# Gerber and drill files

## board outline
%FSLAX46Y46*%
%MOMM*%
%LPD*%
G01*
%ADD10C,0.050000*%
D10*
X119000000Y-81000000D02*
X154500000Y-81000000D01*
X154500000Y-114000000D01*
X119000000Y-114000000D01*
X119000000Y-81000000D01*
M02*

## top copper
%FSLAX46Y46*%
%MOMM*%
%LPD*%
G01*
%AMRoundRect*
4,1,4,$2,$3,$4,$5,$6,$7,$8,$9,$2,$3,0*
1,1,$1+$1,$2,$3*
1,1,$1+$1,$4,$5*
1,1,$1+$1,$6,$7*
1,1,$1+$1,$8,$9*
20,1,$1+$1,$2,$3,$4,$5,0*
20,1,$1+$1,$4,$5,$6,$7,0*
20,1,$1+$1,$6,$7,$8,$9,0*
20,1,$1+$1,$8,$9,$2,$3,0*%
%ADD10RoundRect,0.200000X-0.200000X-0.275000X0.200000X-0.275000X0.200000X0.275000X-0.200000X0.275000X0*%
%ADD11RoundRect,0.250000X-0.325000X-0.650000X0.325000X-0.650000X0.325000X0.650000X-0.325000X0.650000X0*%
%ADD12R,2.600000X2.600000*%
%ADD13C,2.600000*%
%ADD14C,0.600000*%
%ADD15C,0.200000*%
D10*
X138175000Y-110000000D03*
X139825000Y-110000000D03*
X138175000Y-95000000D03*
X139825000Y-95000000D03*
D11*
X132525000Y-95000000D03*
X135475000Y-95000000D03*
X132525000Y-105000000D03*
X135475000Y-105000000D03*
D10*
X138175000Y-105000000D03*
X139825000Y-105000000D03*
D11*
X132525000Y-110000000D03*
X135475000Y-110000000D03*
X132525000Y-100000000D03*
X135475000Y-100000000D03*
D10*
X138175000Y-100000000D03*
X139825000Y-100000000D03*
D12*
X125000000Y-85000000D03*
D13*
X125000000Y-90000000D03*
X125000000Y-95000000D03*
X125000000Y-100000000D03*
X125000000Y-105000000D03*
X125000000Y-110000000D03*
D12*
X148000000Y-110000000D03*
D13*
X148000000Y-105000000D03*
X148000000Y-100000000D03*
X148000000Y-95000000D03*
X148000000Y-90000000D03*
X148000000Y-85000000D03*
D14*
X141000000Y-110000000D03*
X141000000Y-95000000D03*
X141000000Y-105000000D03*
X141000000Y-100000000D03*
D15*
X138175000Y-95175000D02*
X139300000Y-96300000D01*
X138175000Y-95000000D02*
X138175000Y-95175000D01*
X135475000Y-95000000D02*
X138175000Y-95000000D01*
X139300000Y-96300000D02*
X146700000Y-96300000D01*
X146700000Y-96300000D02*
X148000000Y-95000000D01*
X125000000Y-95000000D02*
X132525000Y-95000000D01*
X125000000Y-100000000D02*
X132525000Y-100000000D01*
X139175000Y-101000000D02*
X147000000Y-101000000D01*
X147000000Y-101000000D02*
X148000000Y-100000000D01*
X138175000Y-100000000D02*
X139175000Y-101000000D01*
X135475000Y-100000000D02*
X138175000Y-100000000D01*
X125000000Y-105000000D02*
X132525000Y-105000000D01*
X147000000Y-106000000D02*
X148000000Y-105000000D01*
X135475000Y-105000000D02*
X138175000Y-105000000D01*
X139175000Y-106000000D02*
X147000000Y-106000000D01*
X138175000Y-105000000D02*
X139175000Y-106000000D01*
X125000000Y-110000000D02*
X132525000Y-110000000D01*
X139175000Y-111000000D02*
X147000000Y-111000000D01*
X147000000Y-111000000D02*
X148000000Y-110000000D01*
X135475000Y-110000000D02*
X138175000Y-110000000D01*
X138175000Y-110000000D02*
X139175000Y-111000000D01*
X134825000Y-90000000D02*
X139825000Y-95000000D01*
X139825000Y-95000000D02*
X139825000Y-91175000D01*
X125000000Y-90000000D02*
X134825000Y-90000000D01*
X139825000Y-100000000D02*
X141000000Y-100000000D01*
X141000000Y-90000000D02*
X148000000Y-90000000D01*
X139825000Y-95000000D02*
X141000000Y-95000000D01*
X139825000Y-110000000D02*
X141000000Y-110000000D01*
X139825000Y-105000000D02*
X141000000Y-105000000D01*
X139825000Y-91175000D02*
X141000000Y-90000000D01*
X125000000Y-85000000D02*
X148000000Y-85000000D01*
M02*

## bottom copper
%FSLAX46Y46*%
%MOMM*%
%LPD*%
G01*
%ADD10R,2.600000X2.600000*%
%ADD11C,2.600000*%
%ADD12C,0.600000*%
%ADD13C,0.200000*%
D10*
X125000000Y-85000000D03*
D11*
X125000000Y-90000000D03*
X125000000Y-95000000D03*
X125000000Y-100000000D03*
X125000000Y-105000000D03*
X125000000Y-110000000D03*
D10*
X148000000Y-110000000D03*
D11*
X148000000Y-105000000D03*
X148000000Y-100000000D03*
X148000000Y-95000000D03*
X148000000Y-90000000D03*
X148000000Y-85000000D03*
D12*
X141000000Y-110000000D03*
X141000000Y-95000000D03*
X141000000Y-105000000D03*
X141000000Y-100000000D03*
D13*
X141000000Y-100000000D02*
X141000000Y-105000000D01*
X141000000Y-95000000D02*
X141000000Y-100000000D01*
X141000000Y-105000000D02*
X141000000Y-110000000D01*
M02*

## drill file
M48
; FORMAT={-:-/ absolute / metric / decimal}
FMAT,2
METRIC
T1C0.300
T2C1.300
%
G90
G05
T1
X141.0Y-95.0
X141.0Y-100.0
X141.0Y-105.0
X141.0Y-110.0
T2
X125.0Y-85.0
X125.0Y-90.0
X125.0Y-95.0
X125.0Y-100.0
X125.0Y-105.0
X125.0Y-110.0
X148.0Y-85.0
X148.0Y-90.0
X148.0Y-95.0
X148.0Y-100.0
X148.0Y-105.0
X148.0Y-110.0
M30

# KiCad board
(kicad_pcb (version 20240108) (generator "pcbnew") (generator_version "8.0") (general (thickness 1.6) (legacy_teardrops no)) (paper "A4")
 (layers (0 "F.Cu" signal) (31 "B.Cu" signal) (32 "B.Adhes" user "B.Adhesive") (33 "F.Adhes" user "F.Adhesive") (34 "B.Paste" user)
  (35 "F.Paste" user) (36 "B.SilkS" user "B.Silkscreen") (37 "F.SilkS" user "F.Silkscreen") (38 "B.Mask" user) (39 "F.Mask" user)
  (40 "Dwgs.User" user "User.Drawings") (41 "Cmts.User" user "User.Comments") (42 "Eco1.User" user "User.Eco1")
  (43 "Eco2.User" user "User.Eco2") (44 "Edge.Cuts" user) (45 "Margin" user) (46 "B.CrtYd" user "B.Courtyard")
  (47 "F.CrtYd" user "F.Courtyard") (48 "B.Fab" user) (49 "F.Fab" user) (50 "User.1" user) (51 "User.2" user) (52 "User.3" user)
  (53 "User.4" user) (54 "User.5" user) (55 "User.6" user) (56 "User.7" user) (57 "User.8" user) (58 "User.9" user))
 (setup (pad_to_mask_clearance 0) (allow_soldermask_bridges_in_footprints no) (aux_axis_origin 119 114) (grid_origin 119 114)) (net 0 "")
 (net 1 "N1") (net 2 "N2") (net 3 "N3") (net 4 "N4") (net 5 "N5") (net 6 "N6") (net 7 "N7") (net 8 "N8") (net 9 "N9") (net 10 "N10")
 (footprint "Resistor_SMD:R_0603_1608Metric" (layer "F.Cu") (at 139 110)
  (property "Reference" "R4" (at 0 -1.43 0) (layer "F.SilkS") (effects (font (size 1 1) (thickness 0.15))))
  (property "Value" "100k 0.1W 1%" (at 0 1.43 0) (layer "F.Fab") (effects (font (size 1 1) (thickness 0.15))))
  (pad "1" smd roundrect (at -0.825 0) (size 0.8 0.95) (layers "F.Cu" "F.Paste" "F.Mask") (roundrect_rratio 0.25) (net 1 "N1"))
  (pad "2" smd roundrect (at 0.825 0) (size 0.8 0.95) (layers "F.Cu" "F.Paste" "F.Mask") (roundrect_rratio 0.25) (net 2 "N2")))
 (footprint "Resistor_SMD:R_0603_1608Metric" (layer "F.Cu") (at 139 95)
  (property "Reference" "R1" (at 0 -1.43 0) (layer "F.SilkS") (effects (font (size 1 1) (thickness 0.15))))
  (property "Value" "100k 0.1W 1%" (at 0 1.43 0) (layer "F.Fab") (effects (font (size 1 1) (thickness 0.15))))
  (pad "1" smd roundrect (at -0.825 0) (size 0.8 0.95) (layers "F.Cu" "F.Paste" "F.Mask") (roundrect_rratio 0.25) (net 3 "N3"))
  (pad "2" smd roundrect (at 0.825 0) (size 0.8 0.95) (layers "F.Cu" "F.Paste" "F.Mask") (roundrect_rratio 0.25) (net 2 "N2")))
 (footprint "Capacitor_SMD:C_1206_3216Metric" (layer "F.Cu") (at 134 95)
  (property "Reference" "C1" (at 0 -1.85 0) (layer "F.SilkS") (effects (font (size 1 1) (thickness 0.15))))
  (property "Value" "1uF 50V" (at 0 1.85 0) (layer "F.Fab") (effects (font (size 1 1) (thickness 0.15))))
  (pad "1" smd roundrect (at -1.475 0) (size 1.15 1.8) (layers "F.Cu" "F.Paste" "F.Mask") (roundrect_rratio 0.217391) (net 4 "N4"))
  (pad "2" smd roundrect (at 1.475 0) (size 1.15 1.8) (layers "F.Cu" "F.Paste" "F.Mask") (roundrect_rratio 0.217391) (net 3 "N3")))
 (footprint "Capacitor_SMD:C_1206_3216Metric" (layer "F.Cu") (at 134 105)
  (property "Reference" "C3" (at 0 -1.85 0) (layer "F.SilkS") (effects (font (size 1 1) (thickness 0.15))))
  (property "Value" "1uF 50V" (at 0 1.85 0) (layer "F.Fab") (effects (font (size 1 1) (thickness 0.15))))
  (pad "1" smd roundrect (at -1.475 0) (size 1.15 1.8) (layers "F.Cu" "F.Paste" "F.Mask") (roundrect_rratio 0.217391) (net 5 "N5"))
  (pad "2" smd roundrect (at 1.475 0) (size 1.15 1.8) (layers "F.Cu" "F.Paste" "F.Mask") (roundrect_rratio 0.217391) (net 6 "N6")))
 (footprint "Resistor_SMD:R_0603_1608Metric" (layer "F.Cu") (at 139 105)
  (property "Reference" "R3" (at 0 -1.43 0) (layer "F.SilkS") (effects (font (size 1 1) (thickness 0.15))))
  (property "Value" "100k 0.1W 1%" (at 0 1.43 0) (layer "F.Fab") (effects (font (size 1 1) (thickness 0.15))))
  (pad "1" smd roundrect (at -0.825 0) (size 0.8 0.95) (layers "F.Cu" "F.Paste" "F.Mask") (roundrect_rratio 0.25) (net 6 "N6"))
  (pad "2" smd roundrect (at 0.825 0) (size 0.8 0.95) (layers "F.Cu" "F.Paste" "F.Mask") (roundrect_rratio 0.25) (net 2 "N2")))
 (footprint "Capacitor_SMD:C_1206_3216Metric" (layer "F.Cu") (at 134 110)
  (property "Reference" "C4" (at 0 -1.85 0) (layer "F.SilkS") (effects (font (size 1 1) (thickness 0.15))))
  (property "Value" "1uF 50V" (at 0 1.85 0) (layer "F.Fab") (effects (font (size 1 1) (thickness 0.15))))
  (pad "1" smd roundrect (at -1.475 0) (size 1.15 1.8) (layers "F.Cu" "F.Paste" "F.Mask") (roundrect_rratio 0.217391) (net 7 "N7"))
  (pad "2" smd roundrect (at 1.475 0) (size 1.15 1.8) (layers "F.Cu" "F.Paste" "F.Mask") (roundrect_rratio 0.217391) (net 1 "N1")))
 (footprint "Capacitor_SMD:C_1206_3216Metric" (layer "F.Cu") (at 134 100)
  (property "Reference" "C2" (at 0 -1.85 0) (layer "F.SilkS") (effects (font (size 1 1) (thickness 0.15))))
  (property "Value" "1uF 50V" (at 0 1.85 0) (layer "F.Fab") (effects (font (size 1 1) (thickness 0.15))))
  (pad "1" smd roundrect (at -1.475 0) (size 1.15 1.8) (layers "F.Cu" "F.Paste" "F.Mask") (roundrect_rratio 0.217391) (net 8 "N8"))
  (pad "2" smd roundrect (at 1.475 0) (size 1.15 1.8) (layers "F.Cu" "F.Paste" "F.Mask") (roundrect_rratio 0.217391) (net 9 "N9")))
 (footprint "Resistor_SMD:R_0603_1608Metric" (layer "F.Cu") (at 139 100)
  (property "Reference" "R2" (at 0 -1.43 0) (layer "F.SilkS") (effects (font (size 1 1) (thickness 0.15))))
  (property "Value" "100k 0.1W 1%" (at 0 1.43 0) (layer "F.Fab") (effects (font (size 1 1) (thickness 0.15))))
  (pad "1" smd roundrect (at -0.825 0) (size 0.8 0.95) (layers "F.Cu" "F.Paste" "F.Mask") (roundrect_rratio 0.25) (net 9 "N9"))
  (pad "2" smd roundrect (at 0.825 0) (size 0.8 0.95) (layers "F.Cu" "F.Paste" "F.Mask") (roundrect_rratio 0.25) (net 2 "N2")))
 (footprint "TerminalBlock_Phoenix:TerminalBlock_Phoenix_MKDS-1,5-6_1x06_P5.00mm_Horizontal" (layer "F.Cu") (at 125 85 -90)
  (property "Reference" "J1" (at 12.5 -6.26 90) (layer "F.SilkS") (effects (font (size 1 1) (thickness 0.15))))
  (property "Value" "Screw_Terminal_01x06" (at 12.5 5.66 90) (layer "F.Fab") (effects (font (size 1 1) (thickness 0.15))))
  (pad "1" thru_hole rect (at 0 0 270) (size 2.6 2.6) (drill 1.3) (layers "*.Cu" "*.Mask") (remove_unused_layers no) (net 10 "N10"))
  (pad "2" thru_hole circle (at 5 0 270) (size 2.6 2.6) (drill 1.3) (layers "*.Cu" "*.Mask") (remove_unused_layers no) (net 2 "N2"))
  (pad "3" thru_hole circle (at 10 0 270) (size 2.6 2.6) (drill 1.3) (layers "*.Cu" "*.Mask") (remove_unused_layers no) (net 4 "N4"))
  (pad "4" thru_hole circle (at 15 0 270) (size 2.6 2.6) (drill 1.3) (layers "*.Cu" "*.Mask") (remove_unused_layers no) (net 8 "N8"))
  (pad "5" thru_hole circle (at 20 0 270) (size 2.6 2.6) (drill 1.3) (layers "*.Cu" "*.Mask") (remove_unused_layers no) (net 5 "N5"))
  (pad "6" thru_hole circle (at 25 0 270) (size 2.6 2.6) (drill 1.3) (layers "*.Cu" "*.Mask") (remove_unused_layers no) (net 7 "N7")))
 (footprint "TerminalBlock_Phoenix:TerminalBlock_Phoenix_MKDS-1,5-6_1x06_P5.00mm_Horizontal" (layer "F.Cu") (at 148 110 90)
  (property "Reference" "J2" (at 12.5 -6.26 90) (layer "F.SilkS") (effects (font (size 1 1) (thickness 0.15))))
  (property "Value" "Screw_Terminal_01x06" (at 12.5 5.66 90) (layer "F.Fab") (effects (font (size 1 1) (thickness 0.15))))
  (pad "1" thru_hole rect (at 0 0 90) (size 2.6 2.6) (drill 1.3) (layers "*.Cu" "*.Mask") (remove_unused_layers no) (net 1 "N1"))
  (pad "2" thru_hole circle (at 5 0 90) (size 2.6 2.6) (drill 1.3) (layers "*.Cu" "*.Mask") (remove_unused_layers no) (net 6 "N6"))
  (pad "3" thru_hole circle (at 10 0 90) (size 2.6 2.6) (drill 1.3) (layers "*.Cu" "*.Mask") (remove_unused_layers no) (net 9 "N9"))
  (pad "4" thru_hole circle (at 15 0 90) (size 2.6 2.6) (drill 1.3) (layers "*.Cu" "*.Mask") (remove_unused_layers no) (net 3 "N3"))
  (pad "5" thru_hole circle (at 20 0 90) (size 2.6 2.6) (drill 1.3) (layers "*.Cu" "*.Mask") (remove_unused_layers no) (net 2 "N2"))
  (pad "6" thru_hole circle (at 25 0 90) (size 2.6 2.6) (drill 1.3) (layers "*.Cu" "*.Mask") (remove_unused_layers no) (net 10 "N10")))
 (gr_rect (start 119 81) (end 154.5 114) (stroke (width 0.05) (type default)) (fill none) (layer "Edge.Cuts"))
 (segment (start 138.175 95.175) (end 139.3 96.3) (width 0.2) (layer "F.Cu") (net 3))
 (segment (start 138.175 95) (end 138.175 95.175) (width 0.2) (layer "F.Cu") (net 3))
 (segment (start 135.475 95) (end 138.175 95) (width 0.2) (layer "F.Cu") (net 3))
 (segment (start 139.3 96.3) (end 146.7 96.3) (width 0.2) (layer "F.Cu") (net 3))
 (segment (start 146.7 96.3) (end 148 95) (width 0.2) (layer "F.Cu") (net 3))
 (segment (start 125 95) (end 132.525 95) (width 0.2) (layer "F.Cu") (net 4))
 (segment (start 125 100) (end 132.525 100) (width 0.2) (layer "F.Cu") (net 8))
 (segment (start 139.175 101) (end 147 101) (width 0.2) (layer "F.Cu") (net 9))
 (segment (start 147 101) (end 148 100) (width 0.2) (layer "F.Cu") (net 9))
 (segment (start 138.175 100) (end 139.175 101) (width 0.2) (layer "F.Cu") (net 9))
 (segment (start 135.475 100) (end 138.175 100) (width 0.2) (layer "F.Cu") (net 9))
 (segment (start 125 105) (end 132.525 105) (width 0.2) (layer "F.Cu") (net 5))
 (segment (start 147 106) (end 148 105) (width 0.2) (layer "F.Cu") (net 6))
 (segment (start 135.475 105) (end 138.175 105) (width 0.2) (layer "F.Cu") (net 6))
 (segment (start 139.175 106) (end 147 106) (width 0.2) (layer "F.Cu") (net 6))
 (segment (start 138.175 105) (end 139.175 106) (width 0.2) (layer "F.Cu") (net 6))
 (segment (start 125 110) (end 132.525 110) (width 0.2) (layer "F.Cu") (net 7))
 (segment (start 139.175 111) (end 147 111) (width 0.2) (layer "F.Cu") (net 1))
 (segment (start 147 111) (end 148 110) (width 0.2) (layer "F.Cu") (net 1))
 (segment (start 135.475 110) (end 138.175 110) (width 0.2) (layer "F.Cu") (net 1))
 (segment (start 138.175 110) (end 139.175 111) (width 0.2) (layer "F.Cu") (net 1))
 (segment (start 134.825 90) (end 139.825 95) (width 0.2) (layer "F.Cu") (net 2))
 (segment (start 139.825 95) (end 139.825 91.175) (width 0.2) (layer "F.Cu") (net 2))
 (segment (start 125 90) (end 134.825 90) (width 0.2) (layer "F.Cu") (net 2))
 (segment (start 139.825 100) (end 141 100) (width 0.2) (layer "F.Cu") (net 2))
 (segment (start 141 90) (end 148 90) (width 0.2) (layer "F.Cu") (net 2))
 (segment (start 139.825 95) (end 141 95) (width 0.2) (layer "F.Cu") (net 2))
 (segment (start 139.825 110) (end 141 110) (width 0.2) (layer "F.Cu") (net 2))
 (segment (start 139.825 105) (end 141 105) (width 0.2) (layer "F.Cu") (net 2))
 (segment (start 139.825 91.175) (end 141 90) (width 0.2) (layer "F.Cu") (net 2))
 (via (at 141 110) (size 0.6) (drill 0.3) (layers "F.Cu" "B.Cu") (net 2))
 (via (at 141 95) (size 0.6) (drill 0.3) (layers "F.Cu" "B.Cu") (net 2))
 (via (at 141 105) (size 0.6) (drill 0.3) (layers "F.Cu" "B.Cu") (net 2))
 (via (at 141 100) (size 0.6) (drill 0.3) (layers "F.Cu" "B.Cu") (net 2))
 (segment (start 141 100) (end 141 105) (width 0.2) (layer "B.Cu") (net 2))
 (segment (start 141 95) (end 141 100) (width 0.2) (layer "B.Cu") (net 2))
 (segment (start 141 105) (end 141 110) (width 0.2) (layer "B.Cu") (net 2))
 (segment (start 125 85) (end 148 85) (width 0.2) (layer "F.Cu") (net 10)))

